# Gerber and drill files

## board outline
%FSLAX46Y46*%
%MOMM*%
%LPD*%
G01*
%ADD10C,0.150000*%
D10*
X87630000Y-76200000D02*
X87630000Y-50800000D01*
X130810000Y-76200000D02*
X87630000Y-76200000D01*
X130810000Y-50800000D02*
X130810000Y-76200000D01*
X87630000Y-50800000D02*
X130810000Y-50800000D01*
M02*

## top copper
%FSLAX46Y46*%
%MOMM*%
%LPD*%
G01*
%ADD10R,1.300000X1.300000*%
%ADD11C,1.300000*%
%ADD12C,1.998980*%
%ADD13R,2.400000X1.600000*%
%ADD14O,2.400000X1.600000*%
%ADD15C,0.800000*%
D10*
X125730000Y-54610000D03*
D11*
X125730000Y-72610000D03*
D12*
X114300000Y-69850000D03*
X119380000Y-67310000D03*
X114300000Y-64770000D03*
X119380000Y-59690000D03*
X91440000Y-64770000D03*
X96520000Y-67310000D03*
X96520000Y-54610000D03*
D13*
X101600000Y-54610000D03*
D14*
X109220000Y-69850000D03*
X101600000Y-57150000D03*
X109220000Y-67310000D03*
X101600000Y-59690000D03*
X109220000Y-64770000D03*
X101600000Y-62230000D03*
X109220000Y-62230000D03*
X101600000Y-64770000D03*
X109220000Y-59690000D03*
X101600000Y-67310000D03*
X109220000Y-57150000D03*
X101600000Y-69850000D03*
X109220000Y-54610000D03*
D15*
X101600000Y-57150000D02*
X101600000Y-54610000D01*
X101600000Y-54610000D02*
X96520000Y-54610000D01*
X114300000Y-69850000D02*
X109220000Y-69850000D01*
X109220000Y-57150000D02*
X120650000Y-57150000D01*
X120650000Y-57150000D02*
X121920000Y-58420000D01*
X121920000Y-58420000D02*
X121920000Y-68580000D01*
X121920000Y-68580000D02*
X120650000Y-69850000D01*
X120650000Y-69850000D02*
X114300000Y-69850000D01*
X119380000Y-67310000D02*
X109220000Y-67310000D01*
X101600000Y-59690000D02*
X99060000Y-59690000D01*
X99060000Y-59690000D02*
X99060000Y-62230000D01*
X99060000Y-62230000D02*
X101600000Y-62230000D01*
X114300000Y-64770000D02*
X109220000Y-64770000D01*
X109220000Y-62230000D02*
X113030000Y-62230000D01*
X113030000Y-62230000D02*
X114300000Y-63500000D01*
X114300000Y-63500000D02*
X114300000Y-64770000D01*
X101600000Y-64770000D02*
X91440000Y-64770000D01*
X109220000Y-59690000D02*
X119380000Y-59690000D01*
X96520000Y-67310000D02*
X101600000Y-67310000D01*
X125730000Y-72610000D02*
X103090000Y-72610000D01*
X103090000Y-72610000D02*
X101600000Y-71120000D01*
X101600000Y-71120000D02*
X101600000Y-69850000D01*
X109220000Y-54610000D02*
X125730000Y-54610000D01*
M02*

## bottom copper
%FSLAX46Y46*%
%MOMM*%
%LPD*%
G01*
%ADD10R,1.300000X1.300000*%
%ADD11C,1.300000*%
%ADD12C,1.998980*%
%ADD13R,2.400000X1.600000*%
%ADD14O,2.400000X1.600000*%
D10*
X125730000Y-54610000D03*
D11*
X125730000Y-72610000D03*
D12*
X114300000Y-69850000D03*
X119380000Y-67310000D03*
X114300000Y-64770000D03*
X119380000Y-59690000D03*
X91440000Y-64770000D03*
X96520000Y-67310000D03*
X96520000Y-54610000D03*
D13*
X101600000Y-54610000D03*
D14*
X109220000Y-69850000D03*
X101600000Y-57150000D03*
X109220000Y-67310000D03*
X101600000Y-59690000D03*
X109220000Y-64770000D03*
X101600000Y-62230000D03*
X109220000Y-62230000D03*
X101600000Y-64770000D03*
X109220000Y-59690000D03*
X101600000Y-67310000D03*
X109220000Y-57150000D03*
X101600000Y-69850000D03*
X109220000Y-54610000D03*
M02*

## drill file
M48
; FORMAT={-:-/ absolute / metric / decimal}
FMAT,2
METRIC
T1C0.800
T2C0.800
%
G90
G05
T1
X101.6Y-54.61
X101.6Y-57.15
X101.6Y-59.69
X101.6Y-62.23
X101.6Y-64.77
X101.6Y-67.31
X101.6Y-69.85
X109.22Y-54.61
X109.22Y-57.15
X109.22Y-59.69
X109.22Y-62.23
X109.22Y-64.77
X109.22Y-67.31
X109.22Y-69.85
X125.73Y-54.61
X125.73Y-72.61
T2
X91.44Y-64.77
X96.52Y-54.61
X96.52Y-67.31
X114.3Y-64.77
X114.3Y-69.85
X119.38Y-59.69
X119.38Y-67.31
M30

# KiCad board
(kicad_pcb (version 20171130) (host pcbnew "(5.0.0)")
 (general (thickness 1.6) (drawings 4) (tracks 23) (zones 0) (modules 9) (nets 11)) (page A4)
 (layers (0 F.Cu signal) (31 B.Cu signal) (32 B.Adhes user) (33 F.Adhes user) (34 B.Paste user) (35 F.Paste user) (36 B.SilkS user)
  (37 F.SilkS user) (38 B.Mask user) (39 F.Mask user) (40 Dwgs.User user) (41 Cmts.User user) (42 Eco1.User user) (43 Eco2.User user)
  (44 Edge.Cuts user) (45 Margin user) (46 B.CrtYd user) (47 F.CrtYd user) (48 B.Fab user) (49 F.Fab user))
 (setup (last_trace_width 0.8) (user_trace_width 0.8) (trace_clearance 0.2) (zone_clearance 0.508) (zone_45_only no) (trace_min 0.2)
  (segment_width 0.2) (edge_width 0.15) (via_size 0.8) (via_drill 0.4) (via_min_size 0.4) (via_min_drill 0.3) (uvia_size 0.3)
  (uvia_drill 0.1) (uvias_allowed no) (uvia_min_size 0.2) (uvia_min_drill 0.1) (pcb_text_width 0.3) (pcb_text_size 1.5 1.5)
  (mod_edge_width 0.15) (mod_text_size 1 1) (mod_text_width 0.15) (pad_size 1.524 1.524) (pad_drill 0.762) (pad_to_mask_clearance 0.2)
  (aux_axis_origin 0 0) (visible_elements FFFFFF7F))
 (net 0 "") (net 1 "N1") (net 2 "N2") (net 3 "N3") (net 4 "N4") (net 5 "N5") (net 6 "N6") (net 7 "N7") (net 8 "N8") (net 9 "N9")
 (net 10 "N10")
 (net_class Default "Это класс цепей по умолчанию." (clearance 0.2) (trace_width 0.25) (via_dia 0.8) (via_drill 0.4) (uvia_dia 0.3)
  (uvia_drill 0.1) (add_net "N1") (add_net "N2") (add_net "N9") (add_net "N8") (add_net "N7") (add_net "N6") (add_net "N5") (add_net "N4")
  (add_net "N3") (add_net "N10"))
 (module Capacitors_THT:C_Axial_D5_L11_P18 (layer F.Cu) (at 125.73 54.61 270)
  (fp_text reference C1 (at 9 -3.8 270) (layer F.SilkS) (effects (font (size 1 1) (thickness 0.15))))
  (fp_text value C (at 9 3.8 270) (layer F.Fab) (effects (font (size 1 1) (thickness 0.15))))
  (pad 1 thru_hole rect (at 0 0 270) (size 1.3 1.3) (drill 0.8) (layers *.Cu *.Mask) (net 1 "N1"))
  (pad 2 thru_hole circle (at 18 0 270) (size 1.3 1.3) (drill 0.8) (layers *.Cu *.Mask) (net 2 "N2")))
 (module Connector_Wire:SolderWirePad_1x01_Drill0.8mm (layer F.Cu) (at 114.3 69.85)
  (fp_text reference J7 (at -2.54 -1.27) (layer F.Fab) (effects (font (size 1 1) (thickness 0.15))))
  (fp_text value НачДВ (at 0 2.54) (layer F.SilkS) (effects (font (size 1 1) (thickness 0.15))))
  (pad 1 thru_hole circle (at 0 0) (size 1.99898 1.99898) (drill 0.8001) (layers *.Cu *.Mask) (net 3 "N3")))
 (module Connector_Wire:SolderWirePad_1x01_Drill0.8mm (layer F.Cu) (at 119.38 67.31)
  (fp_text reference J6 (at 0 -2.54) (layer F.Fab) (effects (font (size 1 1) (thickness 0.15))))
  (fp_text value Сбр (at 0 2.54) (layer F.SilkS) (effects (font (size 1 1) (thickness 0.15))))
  (pad 1 thru_hole circle (at 0 0) (size 1.99898 1.99898) (drill 0.8001) (layers *.Cu *.Mask) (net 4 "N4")))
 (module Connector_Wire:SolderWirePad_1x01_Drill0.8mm (layer F.Cu) (at 114.3 64.77)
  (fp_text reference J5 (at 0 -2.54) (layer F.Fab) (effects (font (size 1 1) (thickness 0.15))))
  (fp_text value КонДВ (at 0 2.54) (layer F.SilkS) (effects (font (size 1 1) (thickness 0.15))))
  (pad 1 thru_hole circle (at 0 0) (size 1.99898 1.99898) (drill 0.8001) (layers *.Cu *.Mask) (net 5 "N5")))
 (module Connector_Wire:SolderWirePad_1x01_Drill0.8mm (layer F.Cu) (at 119.38 59.69)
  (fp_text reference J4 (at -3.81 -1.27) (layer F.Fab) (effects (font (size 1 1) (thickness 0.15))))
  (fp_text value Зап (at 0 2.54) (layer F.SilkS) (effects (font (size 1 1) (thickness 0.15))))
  (pad 1 thru_hole circle (at 0 0) (size 1.99898 1.99898) (drill 0.8001) (layers *.Cu *.Mask) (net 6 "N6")))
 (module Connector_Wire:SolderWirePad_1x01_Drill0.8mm (layer F.Cu) (at 91.44 64.77)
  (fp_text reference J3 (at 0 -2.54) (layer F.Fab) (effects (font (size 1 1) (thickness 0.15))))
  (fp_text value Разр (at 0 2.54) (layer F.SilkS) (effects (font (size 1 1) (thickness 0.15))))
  (pad 1 thru_hole circle (at 0 0) (size 1.99898 1.99898) (drill 0.8001) (layers *.Cu *.Mask) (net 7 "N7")))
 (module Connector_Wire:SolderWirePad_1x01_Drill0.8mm (layer F.Cu) (at 96.52 67.31)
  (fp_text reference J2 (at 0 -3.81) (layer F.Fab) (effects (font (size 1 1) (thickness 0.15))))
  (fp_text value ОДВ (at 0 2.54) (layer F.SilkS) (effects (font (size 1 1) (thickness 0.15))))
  (pad 1 thru_hole circle (at 0 0) (size 1.99898 1.99898) (drill 0.8001) (layers *.Cu *.Mask) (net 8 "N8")))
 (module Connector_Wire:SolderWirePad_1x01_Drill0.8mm (layer F.Cu) (at 96.52 54.61)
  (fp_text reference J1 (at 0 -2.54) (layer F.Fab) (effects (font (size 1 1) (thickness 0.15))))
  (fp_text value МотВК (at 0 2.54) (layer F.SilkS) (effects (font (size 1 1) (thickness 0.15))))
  (pad 1 thru_hole circle (at 0 0) (size 1.99898 1.99898) (drill 0.8001) (layers *.Cu *.Mask) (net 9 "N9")))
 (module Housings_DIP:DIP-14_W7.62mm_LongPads (layer F.Cu) (at 101.6 54.61)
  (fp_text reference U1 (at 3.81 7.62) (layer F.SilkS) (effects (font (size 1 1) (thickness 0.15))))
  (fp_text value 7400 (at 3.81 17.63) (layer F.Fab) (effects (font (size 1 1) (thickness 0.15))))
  (pad 1 thru_hole rect (at 0 0) (size 2.4 1.6) (drill 0.8) (layers *.Cu *.Mask) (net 9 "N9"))
  (pad 8 thru_hole oval (at 7.62 15.24) (size 2.4 1.6) (drill 0.8) (layers *.Cu *.Mask) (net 3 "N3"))
  (pad 2 thru_hole oval (at 0 2.54) (size 2.4 1.6) (drill 0.8) (layers *.Cu *.Mask) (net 9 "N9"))
  (pad 9 thru_hole oval (at 7.62 12.7) (size 2.4 1.6) (drill 0.8) (layers *.Cu *.Mask) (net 4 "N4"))
  (pad 3 thru_hole oval (at 0 5.08) (size 2.4 1.6) (drill 0.8) (layers *.Cu *.Mask) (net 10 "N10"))
  (pad 10 thru_hole oval (at 7.62 10.16) (size 2.4 1.6) (drill 0.8) (layers *.Cu *.Mask) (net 5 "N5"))
  (pad 4 thru_hole oval (at 0 7.62) (size 2.4 1.6) (drill 0.8) (layers *.Cu *.Mask) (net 10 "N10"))
  (pad 11 thru_hole oval (at 7.62 7.62) (size 2.4 1.6) (drill 0.8) (layers *.Cu *.Mask) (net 5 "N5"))
  (pad 5 thru_hole oval (at 0 10.16) (size 2.4 1.6) (drill 0.8) (layers *.Cu *.Mask) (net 7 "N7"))
  (pad 12 thru_hole oval (at 7.62 5.08) (size 2.4 1.6) (drill 0.8) (layers *.Cu *.Mask) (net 6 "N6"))
  (pad 6 thru_hole oval (at 0 12.7) (size 2.4 1.6) (drill 0.8) (layers *.Cu *.Mask) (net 8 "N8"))
  (pad 13 thru_hole oval (at 7.62 2.54) (size 2.4 1.6) (drill 0.8) (layers *.Cu *.Mask) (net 3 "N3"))
  (pad 7 thru_hole oval (at 0 15.24) (size 2.4 1.6) (drill 0.8) (layers *.Cu *.Mask) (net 2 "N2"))
  (pad 14 thru_hole oval (at 7.62 0) (size 2.4 1.6) (drill 0.8) (layers *.Cu *.Mask) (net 1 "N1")))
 (gr_line (start 87.63 76.2) (end 87.63 50.8) (layer Edge.Cuts) (width 0.15))
 (gr_line (start 130.81 76.2) (end 87.63 76.2) (layer Edge.Cuts) (width 0.15))
 (gr_line (start 130.81 50.8) (end 130.81 76.2) (layer Edge.Cuts) (width 0.15))
 (gr_line (start 87.63 50.8) (end 130.81 50.8) (layer Edge.Cuts) (width 0.15))
 (segment (start 101.6 57.15) (end 101.6 54.61) (width 0.8) (layer F.Cu) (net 9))
 (segment (start 101.6 54.61) (end 96.52 54.61) (width 0.8) (layer F.Cu) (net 9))
 (segment (start 114.3 69.85) (end 109.22 69.85) (width 0.8) (layer F.Cu) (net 3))
 (segment (start 109.22 57.15) (end 120.65 57.15) (width 0.8) (layer F.Cu) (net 3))
 (segment (start 120.65 57.15) (end 121.92 58.42) (width 0.8) (layer F.Cu) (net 3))
 (segment (start 121.92 58.42) (end 121.92 68.58) (width 0.8) (layer F.Cu) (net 3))
 (segment (start 121.92 68.58) (end 120.65 69.85) (width 0.8) (layer F.Cu) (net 3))
 (segment (start 120.65 69.85) (end 114.3 69.85) (width 0.8) (layer F.Cu) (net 3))
 (segment (start 119.38 67.31) (end 109.22 67.31) (width 0.8) (layer F.Cu) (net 4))
 (segment (start 101.6 59.69) (end 99.06 59.69) (width 0.8) (layer F.Cu) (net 10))
 (segment (start 99.06 59.69) (end 99.06 62.23) (width 0.8) (layer F.Cu) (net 10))
 (segment (start 99.06 62.23) (end 101.6 62.23) (width 0.8) (layer F.Cu) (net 10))
 (segment (start 114.3 64.77) (end 109.22 64.77) (width 0.8) (layer F.Cu) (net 5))
 (segment (start 109.22 62.23) (end 113.03 62.23) (width 0.8) (layer F.Cu) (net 5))
 (segment (start 113.03 62.23) (end 114.3 63.5) (width 0.8) (layer F.Cu) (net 5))
 (segment (start 114.3 63.5) (end 114.3 64.77) (width 0.8) (layer F.Cu) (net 5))
 (segment (start 101.6 64.77) (end 91.44 64.77) (width 0.8) (layer F.Cu) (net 7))
 (segment (start 109.22 59.69) (end 119.38 59.69) (width 0.8) (layer F.Cu) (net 6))
 (segment (start 96.52 67.31) (end 101.6 67.31) (width 0.8) (layer F.Cu) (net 8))
 (segment (start 125.73 72.61) (end 103.09 72.61) (width 0.8) (layer F.Cu) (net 2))
 (segment (start 103.09 72.61) (end 101.6 71.12) (width 0.8) (layer F.Cu) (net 2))
 (segment (start 101.6 71.12) (end 101.6 69.85) (width 0.8) (layer F.Cu) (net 2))
 (segment (start 109.22 54.61) (end 125.73 54.61) (width 0.8) (layer F.Cu) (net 1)))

